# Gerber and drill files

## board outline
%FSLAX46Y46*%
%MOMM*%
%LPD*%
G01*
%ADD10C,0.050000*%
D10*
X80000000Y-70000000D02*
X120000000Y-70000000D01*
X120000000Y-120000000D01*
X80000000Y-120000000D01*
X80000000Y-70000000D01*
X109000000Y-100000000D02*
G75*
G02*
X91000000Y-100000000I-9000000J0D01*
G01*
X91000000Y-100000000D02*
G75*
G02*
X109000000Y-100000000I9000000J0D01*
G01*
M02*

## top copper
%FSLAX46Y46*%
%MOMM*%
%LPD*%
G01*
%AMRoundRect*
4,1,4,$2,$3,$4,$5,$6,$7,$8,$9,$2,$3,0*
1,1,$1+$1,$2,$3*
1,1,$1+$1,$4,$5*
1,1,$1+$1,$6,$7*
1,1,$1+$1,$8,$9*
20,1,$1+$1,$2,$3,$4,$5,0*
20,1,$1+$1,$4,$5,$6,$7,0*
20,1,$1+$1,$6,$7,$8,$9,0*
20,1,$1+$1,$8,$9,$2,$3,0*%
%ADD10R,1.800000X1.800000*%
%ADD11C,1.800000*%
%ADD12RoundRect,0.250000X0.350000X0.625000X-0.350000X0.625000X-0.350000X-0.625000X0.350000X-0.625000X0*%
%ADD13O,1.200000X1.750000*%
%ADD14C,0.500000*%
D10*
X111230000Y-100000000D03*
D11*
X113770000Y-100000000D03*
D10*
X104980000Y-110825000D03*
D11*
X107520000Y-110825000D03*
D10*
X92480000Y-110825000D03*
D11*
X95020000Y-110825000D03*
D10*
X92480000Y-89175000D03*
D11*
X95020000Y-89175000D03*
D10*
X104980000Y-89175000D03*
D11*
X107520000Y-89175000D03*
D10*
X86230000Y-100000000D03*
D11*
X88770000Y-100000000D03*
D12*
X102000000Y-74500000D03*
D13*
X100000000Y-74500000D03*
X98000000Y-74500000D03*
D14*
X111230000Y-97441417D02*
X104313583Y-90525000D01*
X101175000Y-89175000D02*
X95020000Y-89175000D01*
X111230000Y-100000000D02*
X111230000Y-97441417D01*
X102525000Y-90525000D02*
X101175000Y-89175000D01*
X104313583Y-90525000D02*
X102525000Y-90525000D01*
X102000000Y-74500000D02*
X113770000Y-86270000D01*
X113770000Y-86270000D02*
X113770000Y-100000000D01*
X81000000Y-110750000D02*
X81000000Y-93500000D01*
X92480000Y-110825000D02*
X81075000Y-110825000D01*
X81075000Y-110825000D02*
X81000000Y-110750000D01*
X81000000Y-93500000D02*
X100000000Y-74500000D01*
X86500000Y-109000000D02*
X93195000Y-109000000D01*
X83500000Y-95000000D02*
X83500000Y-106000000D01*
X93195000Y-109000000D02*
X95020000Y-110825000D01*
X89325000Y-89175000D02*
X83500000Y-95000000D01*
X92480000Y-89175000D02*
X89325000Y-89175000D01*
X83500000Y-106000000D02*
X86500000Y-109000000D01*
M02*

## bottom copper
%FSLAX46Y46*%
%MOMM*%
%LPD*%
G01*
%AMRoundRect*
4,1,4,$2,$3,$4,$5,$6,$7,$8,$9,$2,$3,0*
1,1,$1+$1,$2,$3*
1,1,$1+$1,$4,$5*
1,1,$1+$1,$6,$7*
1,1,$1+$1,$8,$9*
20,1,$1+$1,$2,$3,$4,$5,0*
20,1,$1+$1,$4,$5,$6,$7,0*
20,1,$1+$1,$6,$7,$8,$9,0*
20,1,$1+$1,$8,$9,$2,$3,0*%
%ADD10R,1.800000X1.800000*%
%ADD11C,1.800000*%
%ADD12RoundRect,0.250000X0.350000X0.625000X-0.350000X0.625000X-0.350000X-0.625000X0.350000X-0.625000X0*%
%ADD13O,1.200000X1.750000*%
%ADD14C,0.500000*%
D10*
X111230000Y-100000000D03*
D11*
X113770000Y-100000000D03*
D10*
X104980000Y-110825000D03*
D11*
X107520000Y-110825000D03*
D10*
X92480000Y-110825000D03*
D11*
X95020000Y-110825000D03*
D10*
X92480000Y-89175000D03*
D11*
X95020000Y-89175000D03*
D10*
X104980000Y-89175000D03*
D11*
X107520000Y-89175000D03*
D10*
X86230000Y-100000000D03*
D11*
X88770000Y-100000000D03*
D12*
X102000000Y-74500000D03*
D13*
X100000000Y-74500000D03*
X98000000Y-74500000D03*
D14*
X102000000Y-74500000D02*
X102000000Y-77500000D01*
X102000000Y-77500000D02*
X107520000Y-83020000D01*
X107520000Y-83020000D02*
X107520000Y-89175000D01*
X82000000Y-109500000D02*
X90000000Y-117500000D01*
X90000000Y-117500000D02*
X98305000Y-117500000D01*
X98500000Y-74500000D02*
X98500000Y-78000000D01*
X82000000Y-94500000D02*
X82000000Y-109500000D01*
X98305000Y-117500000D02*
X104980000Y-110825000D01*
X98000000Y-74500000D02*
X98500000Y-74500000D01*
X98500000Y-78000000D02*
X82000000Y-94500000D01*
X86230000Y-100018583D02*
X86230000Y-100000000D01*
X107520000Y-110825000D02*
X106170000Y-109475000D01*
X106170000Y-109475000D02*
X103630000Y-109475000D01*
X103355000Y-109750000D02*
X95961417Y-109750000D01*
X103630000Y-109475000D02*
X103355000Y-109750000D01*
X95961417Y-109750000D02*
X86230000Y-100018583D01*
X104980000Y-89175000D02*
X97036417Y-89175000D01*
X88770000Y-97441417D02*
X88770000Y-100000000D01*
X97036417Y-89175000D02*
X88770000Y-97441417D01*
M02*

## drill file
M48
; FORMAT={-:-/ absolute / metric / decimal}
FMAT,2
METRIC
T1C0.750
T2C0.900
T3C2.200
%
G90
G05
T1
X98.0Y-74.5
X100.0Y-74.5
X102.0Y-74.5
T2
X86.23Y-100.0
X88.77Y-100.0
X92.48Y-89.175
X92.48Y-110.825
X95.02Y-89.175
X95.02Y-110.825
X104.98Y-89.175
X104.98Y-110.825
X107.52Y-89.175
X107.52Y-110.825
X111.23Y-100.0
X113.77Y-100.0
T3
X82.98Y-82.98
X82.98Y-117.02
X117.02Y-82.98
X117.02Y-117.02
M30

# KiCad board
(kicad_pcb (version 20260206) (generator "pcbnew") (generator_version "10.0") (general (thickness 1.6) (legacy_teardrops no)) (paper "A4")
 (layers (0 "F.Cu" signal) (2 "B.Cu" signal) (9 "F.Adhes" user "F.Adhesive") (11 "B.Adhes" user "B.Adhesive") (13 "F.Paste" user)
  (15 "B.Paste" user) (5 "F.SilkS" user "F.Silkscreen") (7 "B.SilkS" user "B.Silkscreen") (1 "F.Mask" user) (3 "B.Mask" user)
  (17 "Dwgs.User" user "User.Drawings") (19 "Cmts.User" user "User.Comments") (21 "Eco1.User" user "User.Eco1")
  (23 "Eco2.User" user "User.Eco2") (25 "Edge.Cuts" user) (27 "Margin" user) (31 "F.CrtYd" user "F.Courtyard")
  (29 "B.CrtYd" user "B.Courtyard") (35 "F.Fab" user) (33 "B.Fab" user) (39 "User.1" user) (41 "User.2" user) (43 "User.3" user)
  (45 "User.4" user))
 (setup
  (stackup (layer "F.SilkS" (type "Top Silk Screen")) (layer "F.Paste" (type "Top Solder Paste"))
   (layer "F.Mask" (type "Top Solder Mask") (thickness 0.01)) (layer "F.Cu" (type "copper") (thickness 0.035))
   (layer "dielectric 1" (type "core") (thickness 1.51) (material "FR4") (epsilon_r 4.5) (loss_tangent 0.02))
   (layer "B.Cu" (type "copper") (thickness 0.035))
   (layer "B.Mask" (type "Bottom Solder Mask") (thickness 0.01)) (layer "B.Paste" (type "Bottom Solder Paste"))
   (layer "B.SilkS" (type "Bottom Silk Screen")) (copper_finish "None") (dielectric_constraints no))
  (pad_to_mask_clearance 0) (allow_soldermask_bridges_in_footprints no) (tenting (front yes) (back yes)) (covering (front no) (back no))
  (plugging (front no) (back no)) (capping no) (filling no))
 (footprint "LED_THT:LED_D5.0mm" (layer "F.Cu") (at 111.23 100)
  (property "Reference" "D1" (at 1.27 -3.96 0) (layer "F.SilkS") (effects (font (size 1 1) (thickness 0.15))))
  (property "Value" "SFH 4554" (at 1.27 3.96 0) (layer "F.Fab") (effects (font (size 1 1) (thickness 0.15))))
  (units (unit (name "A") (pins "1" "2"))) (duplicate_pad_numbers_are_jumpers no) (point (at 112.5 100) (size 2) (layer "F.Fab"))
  (pad "1" thru_hole rect (at 0 0) (size 1.8 1.8) (drill 0.9) (layers "*.Cu" "*.Mask") (remove_unused_layers no) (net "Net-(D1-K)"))
  (pad "2" thru_hole circle (at 2.54 0) (size 1.8 1.8) (drill 0.9) (layers "*.Cu" "*.Mask") (remove_unused_layers no) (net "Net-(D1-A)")))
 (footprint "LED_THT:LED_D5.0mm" (layer "F.Cu") (at 104.98 110.825)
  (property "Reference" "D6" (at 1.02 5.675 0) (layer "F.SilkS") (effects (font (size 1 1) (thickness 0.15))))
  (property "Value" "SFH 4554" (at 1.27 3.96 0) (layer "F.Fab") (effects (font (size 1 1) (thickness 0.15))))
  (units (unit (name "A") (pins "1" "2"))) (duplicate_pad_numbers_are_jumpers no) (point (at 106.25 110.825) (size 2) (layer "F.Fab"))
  (pad "1" thru_hole rect (at 0 0) (size 1.8 1.8) (drill 0.9) (layers "*.Cu" "*.Mask") (remove_unused_layers no) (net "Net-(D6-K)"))
  (pad "2" thru_hole circle (at 2.54 0) (size 1.8 1.8) (drill 0.9) (layers "*.Cu" "*.Mask") (remove_unused_layers no) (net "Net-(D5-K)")))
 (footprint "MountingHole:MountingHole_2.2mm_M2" (layer "F.Cu") (at 117.02 117.02)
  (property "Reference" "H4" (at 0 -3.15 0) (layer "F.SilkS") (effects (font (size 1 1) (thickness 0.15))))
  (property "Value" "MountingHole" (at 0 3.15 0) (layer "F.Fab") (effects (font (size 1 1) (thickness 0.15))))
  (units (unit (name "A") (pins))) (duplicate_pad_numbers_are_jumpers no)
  (pad "" np_thru_hole circle (at 0 0) (size 2.2 2.2) (drill 2.2) (layers "*.Cu" "*.Mask")))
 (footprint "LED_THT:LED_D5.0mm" (layer "F.Cu") (at 92.48 110.825)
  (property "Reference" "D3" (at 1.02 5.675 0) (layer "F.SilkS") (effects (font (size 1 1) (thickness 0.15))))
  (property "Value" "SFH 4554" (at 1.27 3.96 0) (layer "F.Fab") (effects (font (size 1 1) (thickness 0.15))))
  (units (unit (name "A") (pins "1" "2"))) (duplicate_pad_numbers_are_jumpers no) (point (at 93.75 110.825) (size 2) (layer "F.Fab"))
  (pad "1" thru_hole rect (at 0 0) (size 1.8 1.8) (drill 0.9) (layers "*.Cu" "*.Mask") (remove_unused_layers no) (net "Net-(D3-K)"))
  (pad "2" thru_hole circle (at 2.54 0) (size 1.8 1.8) (drill 0.9) (layers "*.Cu" "*.Mask") (remove_unused_layers no) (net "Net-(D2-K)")))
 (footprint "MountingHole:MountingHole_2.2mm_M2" (layer "F.Cu") (at 82.98 117.02)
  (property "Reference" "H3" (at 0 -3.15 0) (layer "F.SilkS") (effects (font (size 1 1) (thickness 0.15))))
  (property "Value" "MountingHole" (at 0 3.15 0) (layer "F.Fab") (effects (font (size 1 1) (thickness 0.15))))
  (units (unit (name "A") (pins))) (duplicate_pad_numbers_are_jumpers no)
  (pad "" np_thru_hole circle (at 0 0) (size 2.2 2.2) (drill 2.2) (layers "*.Cu" "*.Mask")))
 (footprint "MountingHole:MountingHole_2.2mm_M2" (layer "F.Cu") (at 82.98 82.98)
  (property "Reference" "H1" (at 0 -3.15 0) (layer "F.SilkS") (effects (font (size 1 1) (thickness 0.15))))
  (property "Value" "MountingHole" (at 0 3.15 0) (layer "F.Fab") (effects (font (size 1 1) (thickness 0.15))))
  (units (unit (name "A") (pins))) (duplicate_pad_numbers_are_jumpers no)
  (pad "" np_thru_hole circle (at 0 0) (size 2.2 2.2) (drill 2.2) (layers "*.Cu" "*.Mask")))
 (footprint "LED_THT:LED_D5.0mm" (layer "F.Cu") (at 92.48 89.175)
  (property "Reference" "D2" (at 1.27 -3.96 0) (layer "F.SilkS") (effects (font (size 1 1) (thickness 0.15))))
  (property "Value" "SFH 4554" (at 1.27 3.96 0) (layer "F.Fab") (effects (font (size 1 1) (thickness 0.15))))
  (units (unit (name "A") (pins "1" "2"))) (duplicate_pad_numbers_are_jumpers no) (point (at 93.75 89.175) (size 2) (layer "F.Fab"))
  (pad "1" thru_hole rect (at 0 0) (size 1.8 1.8) (drill 0.9) (layers "*.Cu" "*.Mask") (remove_unused_layers no) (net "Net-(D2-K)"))
  (pad "2" thru_hole circle (at 2.54 0) (size 1.8 1.8) (drill 0.9) (layers "*.Cu" "*.Mask") (remove_unused_layers no) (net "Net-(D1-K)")))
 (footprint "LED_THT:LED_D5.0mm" (layer "F.Cu") (at 104.98 89.175)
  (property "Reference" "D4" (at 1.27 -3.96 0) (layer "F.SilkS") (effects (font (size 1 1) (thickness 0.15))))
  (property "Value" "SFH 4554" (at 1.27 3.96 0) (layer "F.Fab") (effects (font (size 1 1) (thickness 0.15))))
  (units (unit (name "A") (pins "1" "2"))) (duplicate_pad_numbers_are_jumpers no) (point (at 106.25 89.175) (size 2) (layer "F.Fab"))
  (pad "1" thru_hole rect (at 0 0) (size 1.8 1.8) (drill 0.9) (layers "*.Cu" "*.Mask") (remove_unused_layers no) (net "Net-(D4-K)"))
  (pad "2" thru_hole circle (at 2.54 0) (size 1.8 1.8) (drill 0.9) (layers "*.Cu" "*.Mask") (remove_unused_layers no) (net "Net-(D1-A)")))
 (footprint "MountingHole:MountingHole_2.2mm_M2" (layer "F.Cu") (at 117.02 82.98)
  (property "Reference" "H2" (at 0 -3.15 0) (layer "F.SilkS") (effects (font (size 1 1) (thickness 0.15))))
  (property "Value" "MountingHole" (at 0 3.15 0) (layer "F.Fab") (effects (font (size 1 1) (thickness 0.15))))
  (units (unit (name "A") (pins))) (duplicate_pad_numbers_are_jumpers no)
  (pad "" np_thru_hole circle (at 0 0) (size 2.2 2.2) (drill 2.2) (layers "*.Cu" "*.Mask")))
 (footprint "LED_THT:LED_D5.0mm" (layer "F.Cu") (at 86.23 100)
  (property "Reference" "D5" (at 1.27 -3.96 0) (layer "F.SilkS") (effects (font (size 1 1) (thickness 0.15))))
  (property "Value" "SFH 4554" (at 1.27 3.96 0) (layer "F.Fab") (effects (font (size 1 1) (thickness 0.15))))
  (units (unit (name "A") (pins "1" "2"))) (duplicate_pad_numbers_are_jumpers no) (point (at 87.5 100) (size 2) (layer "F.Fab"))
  (pad "1" thru_hole rect (at 0 0) (size 1.8 1.8) (drill 0.9) (layers "*.Cu" "*.Mask") (remove_unused_layers no) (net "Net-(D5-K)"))
  (pad "2" thru_hole circle (at 2.54 0) (size 1.8 1.8) (drill 0.9) (layers "*.Cu" "*.Mask") (remove_unused_layers no) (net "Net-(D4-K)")))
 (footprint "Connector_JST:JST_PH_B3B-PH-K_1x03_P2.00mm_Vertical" (layer "B.Cu") (at 102 74.5 180)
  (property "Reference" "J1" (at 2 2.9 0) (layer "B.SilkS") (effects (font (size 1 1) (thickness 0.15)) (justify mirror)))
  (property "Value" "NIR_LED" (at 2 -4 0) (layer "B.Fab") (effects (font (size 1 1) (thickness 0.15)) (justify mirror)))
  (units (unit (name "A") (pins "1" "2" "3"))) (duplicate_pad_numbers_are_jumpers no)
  (pad "1" thru_hole roundrect (at 0 0 180) (size 1.2 1.75) (drill 0.75) (layers "*.Cu" "*.Mask") (remove_unused_layers no)
   (roundrect_rratio 0.208333) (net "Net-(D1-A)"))
  (pad "2" thru_hole oval (at 2 0 180) (size 1.2 1.75) (drill 0.75) (layers "*.Cu" "*.Mask") (remove_unused_layers no) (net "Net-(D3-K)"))
  (pad "3" thru_hole oval (at 4 0 180) (size 1.2 1.75) (drill 0.75) (layers "*.Cu" "*.Mask") (remove_unused_layers no) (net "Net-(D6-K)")))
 (gr_rect (start 80 70) (end 120 120) (stroke (width 0.05) (type solid)) (fill no) (layer "Edge.Cuts"))
 (gr_circle (center 100 100) (end 109 100) (stroke (width 0.05) (type solid)) (fill no) (layer "Edge.Cuts"))
 (segment (start 111.23 97.441417) (end 104.313583 90.525) (width 0.5) (layer "F.Cu") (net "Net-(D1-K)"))
 (segment (start 101.175 89.175) (end 95.02 89.175) (width 0.5) (layer "F.Cu") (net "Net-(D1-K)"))
 (segment (start 111.23 100) (end 111.23 97.441417) (width 0.5) (layer "F.Cu") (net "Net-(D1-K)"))
 (segment (start 102.525 90.525) (end 101.175 89.175) (width 0.5) (layer "F.Cu") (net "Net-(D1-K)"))
 (segment (start 104.313583 90.525) (end 102.525 90.525) (width 0.5) (layer "F.Cu") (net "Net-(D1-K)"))
 (segment (start 102 74.5) (end 113.77 86.27) (width 0.5) (layer "F.Cu") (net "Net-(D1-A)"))
 (segment (start 113.77 86.27) (end 113.77 100) (width 0.5) (layer "F.Cu") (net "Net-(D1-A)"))
 (segment (start 102 74.5) (end 102 77.5) (width 0.5) (layer "B.Cu") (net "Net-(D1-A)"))
 (segment (start 102 77.5) (end 107.52 83.02) (width 0.5) (layer "B.Cu") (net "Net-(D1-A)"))
 (segment (start 107.52 83.02) (end 107.52 89.175) (width 0.5) (layer "B.Cu") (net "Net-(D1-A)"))
 (segment (start 82 109.5) (end 90 117.5) (width 0.5) (layer "B.Cu") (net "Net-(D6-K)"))
 (segment (start 90 117.5) (end 98.305 117.5) (width 0.5) (layer "B.Cu") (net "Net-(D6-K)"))
 (segment (start 98.5 74.5) (end 98.5 78) (width 0.5) (layer "B.Cu") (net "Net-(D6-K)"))
 (segment (start 82 94.5) (end 82 109.5) (width 0.5) (layer "B.Cu") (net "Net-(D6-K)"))
 (segment (start 98.305 117.5) (end 104.98 110.825) (width 0.5) (layer "B.Cu") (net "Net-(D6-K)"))
 (segment (start 98 74.5) (end 98.5 74.5) (width 0.5) (layer "B.Cu") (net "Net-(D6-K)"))
 (segment (start 98.5 78) (end 82 94.5) (width 0.5) (layer "B.Cu") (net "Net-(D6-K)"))
 (segment (start 86.23 100.018583) (end 86.23 100) (width 0.5) (layer "B.Cu") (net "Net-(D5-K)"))
 (segment (start 107.52 110.825) (end 106.17 109.475) (width 0.5) (layer "B.Cu") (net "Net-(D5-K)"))
 (segment (start 106.17 109.475) (end 103.63 109.475) (width 0.5) (layer "B.Cu") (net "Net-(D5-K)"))
 (segment (start 103.355 109.75) (end 95.961417 109.75) (width 0.5) (layer "B.Cu") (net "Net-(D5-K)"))
 (segment (start 103.63 109.475) (end 103.355 109.75) (width 0.5) (layer "B.Cu") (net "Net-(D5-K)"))
 (segment (start 95.961417 109.75) (end 86.23 100.018583) (width 0.5) (layer "B.Cu") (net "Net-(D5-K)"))
 (segment (start 81 110.75) (end 81 93.5) (width 0.5) (layer "F.Cu") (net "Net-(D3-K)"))
 (segment (start 92.48 110.825) (end 81.075 110.825) (width 0.5) (layer "F.Cu") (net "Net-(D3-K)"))
 (segment (start 81.075 110.825) (end 81 110.75) (width 0.5) (layer "F.Cu") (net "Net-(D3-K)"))
 (segment (start 81 93.5) (end 100 74.5) (width 0.5) (layer "F.Cu") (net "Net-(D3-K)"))
 (segment (start 86.5 109) (end 93.195 109) (width 0.5) (layer "F.Cu") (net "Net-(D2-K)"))
 (segment (start 83.5 95) (end 83.5 106) (width 0.5) (layer "F.Cu") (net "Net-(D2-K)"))
 (segment (start 93.195 109) (end 95.02 110.825) (width 0.5) (layer "F.Cu") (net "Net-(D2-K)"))
 (segment (start 89.325 89.175) (end 83.5 95) (width 0.5) (layer "F.Cu") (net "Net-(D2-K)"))
 (segment (start 92.48 89.175) (end 89.325 89.175) (width 0.5) (layer "F.Cu") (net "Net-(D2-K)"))
 (segment (start 83.5 106) (end 86.5 109) (width 0.5) (layer "F.Cu") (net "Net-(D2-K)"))
 (segment (start 104.98 89.175) (end 97.036417 89.175) (width 0.5) (layer "B.Cu") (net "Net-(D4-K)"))
 (segment (start 88.77 97.441417) (end 88.77 100) (width 0.5) (layer "B.Cu") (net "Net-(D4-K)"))
 (segment (start 97.036417 89.175) (end 88.77 97.441417) (width 0.5) (layer "B.Cu") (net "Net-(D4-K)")))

